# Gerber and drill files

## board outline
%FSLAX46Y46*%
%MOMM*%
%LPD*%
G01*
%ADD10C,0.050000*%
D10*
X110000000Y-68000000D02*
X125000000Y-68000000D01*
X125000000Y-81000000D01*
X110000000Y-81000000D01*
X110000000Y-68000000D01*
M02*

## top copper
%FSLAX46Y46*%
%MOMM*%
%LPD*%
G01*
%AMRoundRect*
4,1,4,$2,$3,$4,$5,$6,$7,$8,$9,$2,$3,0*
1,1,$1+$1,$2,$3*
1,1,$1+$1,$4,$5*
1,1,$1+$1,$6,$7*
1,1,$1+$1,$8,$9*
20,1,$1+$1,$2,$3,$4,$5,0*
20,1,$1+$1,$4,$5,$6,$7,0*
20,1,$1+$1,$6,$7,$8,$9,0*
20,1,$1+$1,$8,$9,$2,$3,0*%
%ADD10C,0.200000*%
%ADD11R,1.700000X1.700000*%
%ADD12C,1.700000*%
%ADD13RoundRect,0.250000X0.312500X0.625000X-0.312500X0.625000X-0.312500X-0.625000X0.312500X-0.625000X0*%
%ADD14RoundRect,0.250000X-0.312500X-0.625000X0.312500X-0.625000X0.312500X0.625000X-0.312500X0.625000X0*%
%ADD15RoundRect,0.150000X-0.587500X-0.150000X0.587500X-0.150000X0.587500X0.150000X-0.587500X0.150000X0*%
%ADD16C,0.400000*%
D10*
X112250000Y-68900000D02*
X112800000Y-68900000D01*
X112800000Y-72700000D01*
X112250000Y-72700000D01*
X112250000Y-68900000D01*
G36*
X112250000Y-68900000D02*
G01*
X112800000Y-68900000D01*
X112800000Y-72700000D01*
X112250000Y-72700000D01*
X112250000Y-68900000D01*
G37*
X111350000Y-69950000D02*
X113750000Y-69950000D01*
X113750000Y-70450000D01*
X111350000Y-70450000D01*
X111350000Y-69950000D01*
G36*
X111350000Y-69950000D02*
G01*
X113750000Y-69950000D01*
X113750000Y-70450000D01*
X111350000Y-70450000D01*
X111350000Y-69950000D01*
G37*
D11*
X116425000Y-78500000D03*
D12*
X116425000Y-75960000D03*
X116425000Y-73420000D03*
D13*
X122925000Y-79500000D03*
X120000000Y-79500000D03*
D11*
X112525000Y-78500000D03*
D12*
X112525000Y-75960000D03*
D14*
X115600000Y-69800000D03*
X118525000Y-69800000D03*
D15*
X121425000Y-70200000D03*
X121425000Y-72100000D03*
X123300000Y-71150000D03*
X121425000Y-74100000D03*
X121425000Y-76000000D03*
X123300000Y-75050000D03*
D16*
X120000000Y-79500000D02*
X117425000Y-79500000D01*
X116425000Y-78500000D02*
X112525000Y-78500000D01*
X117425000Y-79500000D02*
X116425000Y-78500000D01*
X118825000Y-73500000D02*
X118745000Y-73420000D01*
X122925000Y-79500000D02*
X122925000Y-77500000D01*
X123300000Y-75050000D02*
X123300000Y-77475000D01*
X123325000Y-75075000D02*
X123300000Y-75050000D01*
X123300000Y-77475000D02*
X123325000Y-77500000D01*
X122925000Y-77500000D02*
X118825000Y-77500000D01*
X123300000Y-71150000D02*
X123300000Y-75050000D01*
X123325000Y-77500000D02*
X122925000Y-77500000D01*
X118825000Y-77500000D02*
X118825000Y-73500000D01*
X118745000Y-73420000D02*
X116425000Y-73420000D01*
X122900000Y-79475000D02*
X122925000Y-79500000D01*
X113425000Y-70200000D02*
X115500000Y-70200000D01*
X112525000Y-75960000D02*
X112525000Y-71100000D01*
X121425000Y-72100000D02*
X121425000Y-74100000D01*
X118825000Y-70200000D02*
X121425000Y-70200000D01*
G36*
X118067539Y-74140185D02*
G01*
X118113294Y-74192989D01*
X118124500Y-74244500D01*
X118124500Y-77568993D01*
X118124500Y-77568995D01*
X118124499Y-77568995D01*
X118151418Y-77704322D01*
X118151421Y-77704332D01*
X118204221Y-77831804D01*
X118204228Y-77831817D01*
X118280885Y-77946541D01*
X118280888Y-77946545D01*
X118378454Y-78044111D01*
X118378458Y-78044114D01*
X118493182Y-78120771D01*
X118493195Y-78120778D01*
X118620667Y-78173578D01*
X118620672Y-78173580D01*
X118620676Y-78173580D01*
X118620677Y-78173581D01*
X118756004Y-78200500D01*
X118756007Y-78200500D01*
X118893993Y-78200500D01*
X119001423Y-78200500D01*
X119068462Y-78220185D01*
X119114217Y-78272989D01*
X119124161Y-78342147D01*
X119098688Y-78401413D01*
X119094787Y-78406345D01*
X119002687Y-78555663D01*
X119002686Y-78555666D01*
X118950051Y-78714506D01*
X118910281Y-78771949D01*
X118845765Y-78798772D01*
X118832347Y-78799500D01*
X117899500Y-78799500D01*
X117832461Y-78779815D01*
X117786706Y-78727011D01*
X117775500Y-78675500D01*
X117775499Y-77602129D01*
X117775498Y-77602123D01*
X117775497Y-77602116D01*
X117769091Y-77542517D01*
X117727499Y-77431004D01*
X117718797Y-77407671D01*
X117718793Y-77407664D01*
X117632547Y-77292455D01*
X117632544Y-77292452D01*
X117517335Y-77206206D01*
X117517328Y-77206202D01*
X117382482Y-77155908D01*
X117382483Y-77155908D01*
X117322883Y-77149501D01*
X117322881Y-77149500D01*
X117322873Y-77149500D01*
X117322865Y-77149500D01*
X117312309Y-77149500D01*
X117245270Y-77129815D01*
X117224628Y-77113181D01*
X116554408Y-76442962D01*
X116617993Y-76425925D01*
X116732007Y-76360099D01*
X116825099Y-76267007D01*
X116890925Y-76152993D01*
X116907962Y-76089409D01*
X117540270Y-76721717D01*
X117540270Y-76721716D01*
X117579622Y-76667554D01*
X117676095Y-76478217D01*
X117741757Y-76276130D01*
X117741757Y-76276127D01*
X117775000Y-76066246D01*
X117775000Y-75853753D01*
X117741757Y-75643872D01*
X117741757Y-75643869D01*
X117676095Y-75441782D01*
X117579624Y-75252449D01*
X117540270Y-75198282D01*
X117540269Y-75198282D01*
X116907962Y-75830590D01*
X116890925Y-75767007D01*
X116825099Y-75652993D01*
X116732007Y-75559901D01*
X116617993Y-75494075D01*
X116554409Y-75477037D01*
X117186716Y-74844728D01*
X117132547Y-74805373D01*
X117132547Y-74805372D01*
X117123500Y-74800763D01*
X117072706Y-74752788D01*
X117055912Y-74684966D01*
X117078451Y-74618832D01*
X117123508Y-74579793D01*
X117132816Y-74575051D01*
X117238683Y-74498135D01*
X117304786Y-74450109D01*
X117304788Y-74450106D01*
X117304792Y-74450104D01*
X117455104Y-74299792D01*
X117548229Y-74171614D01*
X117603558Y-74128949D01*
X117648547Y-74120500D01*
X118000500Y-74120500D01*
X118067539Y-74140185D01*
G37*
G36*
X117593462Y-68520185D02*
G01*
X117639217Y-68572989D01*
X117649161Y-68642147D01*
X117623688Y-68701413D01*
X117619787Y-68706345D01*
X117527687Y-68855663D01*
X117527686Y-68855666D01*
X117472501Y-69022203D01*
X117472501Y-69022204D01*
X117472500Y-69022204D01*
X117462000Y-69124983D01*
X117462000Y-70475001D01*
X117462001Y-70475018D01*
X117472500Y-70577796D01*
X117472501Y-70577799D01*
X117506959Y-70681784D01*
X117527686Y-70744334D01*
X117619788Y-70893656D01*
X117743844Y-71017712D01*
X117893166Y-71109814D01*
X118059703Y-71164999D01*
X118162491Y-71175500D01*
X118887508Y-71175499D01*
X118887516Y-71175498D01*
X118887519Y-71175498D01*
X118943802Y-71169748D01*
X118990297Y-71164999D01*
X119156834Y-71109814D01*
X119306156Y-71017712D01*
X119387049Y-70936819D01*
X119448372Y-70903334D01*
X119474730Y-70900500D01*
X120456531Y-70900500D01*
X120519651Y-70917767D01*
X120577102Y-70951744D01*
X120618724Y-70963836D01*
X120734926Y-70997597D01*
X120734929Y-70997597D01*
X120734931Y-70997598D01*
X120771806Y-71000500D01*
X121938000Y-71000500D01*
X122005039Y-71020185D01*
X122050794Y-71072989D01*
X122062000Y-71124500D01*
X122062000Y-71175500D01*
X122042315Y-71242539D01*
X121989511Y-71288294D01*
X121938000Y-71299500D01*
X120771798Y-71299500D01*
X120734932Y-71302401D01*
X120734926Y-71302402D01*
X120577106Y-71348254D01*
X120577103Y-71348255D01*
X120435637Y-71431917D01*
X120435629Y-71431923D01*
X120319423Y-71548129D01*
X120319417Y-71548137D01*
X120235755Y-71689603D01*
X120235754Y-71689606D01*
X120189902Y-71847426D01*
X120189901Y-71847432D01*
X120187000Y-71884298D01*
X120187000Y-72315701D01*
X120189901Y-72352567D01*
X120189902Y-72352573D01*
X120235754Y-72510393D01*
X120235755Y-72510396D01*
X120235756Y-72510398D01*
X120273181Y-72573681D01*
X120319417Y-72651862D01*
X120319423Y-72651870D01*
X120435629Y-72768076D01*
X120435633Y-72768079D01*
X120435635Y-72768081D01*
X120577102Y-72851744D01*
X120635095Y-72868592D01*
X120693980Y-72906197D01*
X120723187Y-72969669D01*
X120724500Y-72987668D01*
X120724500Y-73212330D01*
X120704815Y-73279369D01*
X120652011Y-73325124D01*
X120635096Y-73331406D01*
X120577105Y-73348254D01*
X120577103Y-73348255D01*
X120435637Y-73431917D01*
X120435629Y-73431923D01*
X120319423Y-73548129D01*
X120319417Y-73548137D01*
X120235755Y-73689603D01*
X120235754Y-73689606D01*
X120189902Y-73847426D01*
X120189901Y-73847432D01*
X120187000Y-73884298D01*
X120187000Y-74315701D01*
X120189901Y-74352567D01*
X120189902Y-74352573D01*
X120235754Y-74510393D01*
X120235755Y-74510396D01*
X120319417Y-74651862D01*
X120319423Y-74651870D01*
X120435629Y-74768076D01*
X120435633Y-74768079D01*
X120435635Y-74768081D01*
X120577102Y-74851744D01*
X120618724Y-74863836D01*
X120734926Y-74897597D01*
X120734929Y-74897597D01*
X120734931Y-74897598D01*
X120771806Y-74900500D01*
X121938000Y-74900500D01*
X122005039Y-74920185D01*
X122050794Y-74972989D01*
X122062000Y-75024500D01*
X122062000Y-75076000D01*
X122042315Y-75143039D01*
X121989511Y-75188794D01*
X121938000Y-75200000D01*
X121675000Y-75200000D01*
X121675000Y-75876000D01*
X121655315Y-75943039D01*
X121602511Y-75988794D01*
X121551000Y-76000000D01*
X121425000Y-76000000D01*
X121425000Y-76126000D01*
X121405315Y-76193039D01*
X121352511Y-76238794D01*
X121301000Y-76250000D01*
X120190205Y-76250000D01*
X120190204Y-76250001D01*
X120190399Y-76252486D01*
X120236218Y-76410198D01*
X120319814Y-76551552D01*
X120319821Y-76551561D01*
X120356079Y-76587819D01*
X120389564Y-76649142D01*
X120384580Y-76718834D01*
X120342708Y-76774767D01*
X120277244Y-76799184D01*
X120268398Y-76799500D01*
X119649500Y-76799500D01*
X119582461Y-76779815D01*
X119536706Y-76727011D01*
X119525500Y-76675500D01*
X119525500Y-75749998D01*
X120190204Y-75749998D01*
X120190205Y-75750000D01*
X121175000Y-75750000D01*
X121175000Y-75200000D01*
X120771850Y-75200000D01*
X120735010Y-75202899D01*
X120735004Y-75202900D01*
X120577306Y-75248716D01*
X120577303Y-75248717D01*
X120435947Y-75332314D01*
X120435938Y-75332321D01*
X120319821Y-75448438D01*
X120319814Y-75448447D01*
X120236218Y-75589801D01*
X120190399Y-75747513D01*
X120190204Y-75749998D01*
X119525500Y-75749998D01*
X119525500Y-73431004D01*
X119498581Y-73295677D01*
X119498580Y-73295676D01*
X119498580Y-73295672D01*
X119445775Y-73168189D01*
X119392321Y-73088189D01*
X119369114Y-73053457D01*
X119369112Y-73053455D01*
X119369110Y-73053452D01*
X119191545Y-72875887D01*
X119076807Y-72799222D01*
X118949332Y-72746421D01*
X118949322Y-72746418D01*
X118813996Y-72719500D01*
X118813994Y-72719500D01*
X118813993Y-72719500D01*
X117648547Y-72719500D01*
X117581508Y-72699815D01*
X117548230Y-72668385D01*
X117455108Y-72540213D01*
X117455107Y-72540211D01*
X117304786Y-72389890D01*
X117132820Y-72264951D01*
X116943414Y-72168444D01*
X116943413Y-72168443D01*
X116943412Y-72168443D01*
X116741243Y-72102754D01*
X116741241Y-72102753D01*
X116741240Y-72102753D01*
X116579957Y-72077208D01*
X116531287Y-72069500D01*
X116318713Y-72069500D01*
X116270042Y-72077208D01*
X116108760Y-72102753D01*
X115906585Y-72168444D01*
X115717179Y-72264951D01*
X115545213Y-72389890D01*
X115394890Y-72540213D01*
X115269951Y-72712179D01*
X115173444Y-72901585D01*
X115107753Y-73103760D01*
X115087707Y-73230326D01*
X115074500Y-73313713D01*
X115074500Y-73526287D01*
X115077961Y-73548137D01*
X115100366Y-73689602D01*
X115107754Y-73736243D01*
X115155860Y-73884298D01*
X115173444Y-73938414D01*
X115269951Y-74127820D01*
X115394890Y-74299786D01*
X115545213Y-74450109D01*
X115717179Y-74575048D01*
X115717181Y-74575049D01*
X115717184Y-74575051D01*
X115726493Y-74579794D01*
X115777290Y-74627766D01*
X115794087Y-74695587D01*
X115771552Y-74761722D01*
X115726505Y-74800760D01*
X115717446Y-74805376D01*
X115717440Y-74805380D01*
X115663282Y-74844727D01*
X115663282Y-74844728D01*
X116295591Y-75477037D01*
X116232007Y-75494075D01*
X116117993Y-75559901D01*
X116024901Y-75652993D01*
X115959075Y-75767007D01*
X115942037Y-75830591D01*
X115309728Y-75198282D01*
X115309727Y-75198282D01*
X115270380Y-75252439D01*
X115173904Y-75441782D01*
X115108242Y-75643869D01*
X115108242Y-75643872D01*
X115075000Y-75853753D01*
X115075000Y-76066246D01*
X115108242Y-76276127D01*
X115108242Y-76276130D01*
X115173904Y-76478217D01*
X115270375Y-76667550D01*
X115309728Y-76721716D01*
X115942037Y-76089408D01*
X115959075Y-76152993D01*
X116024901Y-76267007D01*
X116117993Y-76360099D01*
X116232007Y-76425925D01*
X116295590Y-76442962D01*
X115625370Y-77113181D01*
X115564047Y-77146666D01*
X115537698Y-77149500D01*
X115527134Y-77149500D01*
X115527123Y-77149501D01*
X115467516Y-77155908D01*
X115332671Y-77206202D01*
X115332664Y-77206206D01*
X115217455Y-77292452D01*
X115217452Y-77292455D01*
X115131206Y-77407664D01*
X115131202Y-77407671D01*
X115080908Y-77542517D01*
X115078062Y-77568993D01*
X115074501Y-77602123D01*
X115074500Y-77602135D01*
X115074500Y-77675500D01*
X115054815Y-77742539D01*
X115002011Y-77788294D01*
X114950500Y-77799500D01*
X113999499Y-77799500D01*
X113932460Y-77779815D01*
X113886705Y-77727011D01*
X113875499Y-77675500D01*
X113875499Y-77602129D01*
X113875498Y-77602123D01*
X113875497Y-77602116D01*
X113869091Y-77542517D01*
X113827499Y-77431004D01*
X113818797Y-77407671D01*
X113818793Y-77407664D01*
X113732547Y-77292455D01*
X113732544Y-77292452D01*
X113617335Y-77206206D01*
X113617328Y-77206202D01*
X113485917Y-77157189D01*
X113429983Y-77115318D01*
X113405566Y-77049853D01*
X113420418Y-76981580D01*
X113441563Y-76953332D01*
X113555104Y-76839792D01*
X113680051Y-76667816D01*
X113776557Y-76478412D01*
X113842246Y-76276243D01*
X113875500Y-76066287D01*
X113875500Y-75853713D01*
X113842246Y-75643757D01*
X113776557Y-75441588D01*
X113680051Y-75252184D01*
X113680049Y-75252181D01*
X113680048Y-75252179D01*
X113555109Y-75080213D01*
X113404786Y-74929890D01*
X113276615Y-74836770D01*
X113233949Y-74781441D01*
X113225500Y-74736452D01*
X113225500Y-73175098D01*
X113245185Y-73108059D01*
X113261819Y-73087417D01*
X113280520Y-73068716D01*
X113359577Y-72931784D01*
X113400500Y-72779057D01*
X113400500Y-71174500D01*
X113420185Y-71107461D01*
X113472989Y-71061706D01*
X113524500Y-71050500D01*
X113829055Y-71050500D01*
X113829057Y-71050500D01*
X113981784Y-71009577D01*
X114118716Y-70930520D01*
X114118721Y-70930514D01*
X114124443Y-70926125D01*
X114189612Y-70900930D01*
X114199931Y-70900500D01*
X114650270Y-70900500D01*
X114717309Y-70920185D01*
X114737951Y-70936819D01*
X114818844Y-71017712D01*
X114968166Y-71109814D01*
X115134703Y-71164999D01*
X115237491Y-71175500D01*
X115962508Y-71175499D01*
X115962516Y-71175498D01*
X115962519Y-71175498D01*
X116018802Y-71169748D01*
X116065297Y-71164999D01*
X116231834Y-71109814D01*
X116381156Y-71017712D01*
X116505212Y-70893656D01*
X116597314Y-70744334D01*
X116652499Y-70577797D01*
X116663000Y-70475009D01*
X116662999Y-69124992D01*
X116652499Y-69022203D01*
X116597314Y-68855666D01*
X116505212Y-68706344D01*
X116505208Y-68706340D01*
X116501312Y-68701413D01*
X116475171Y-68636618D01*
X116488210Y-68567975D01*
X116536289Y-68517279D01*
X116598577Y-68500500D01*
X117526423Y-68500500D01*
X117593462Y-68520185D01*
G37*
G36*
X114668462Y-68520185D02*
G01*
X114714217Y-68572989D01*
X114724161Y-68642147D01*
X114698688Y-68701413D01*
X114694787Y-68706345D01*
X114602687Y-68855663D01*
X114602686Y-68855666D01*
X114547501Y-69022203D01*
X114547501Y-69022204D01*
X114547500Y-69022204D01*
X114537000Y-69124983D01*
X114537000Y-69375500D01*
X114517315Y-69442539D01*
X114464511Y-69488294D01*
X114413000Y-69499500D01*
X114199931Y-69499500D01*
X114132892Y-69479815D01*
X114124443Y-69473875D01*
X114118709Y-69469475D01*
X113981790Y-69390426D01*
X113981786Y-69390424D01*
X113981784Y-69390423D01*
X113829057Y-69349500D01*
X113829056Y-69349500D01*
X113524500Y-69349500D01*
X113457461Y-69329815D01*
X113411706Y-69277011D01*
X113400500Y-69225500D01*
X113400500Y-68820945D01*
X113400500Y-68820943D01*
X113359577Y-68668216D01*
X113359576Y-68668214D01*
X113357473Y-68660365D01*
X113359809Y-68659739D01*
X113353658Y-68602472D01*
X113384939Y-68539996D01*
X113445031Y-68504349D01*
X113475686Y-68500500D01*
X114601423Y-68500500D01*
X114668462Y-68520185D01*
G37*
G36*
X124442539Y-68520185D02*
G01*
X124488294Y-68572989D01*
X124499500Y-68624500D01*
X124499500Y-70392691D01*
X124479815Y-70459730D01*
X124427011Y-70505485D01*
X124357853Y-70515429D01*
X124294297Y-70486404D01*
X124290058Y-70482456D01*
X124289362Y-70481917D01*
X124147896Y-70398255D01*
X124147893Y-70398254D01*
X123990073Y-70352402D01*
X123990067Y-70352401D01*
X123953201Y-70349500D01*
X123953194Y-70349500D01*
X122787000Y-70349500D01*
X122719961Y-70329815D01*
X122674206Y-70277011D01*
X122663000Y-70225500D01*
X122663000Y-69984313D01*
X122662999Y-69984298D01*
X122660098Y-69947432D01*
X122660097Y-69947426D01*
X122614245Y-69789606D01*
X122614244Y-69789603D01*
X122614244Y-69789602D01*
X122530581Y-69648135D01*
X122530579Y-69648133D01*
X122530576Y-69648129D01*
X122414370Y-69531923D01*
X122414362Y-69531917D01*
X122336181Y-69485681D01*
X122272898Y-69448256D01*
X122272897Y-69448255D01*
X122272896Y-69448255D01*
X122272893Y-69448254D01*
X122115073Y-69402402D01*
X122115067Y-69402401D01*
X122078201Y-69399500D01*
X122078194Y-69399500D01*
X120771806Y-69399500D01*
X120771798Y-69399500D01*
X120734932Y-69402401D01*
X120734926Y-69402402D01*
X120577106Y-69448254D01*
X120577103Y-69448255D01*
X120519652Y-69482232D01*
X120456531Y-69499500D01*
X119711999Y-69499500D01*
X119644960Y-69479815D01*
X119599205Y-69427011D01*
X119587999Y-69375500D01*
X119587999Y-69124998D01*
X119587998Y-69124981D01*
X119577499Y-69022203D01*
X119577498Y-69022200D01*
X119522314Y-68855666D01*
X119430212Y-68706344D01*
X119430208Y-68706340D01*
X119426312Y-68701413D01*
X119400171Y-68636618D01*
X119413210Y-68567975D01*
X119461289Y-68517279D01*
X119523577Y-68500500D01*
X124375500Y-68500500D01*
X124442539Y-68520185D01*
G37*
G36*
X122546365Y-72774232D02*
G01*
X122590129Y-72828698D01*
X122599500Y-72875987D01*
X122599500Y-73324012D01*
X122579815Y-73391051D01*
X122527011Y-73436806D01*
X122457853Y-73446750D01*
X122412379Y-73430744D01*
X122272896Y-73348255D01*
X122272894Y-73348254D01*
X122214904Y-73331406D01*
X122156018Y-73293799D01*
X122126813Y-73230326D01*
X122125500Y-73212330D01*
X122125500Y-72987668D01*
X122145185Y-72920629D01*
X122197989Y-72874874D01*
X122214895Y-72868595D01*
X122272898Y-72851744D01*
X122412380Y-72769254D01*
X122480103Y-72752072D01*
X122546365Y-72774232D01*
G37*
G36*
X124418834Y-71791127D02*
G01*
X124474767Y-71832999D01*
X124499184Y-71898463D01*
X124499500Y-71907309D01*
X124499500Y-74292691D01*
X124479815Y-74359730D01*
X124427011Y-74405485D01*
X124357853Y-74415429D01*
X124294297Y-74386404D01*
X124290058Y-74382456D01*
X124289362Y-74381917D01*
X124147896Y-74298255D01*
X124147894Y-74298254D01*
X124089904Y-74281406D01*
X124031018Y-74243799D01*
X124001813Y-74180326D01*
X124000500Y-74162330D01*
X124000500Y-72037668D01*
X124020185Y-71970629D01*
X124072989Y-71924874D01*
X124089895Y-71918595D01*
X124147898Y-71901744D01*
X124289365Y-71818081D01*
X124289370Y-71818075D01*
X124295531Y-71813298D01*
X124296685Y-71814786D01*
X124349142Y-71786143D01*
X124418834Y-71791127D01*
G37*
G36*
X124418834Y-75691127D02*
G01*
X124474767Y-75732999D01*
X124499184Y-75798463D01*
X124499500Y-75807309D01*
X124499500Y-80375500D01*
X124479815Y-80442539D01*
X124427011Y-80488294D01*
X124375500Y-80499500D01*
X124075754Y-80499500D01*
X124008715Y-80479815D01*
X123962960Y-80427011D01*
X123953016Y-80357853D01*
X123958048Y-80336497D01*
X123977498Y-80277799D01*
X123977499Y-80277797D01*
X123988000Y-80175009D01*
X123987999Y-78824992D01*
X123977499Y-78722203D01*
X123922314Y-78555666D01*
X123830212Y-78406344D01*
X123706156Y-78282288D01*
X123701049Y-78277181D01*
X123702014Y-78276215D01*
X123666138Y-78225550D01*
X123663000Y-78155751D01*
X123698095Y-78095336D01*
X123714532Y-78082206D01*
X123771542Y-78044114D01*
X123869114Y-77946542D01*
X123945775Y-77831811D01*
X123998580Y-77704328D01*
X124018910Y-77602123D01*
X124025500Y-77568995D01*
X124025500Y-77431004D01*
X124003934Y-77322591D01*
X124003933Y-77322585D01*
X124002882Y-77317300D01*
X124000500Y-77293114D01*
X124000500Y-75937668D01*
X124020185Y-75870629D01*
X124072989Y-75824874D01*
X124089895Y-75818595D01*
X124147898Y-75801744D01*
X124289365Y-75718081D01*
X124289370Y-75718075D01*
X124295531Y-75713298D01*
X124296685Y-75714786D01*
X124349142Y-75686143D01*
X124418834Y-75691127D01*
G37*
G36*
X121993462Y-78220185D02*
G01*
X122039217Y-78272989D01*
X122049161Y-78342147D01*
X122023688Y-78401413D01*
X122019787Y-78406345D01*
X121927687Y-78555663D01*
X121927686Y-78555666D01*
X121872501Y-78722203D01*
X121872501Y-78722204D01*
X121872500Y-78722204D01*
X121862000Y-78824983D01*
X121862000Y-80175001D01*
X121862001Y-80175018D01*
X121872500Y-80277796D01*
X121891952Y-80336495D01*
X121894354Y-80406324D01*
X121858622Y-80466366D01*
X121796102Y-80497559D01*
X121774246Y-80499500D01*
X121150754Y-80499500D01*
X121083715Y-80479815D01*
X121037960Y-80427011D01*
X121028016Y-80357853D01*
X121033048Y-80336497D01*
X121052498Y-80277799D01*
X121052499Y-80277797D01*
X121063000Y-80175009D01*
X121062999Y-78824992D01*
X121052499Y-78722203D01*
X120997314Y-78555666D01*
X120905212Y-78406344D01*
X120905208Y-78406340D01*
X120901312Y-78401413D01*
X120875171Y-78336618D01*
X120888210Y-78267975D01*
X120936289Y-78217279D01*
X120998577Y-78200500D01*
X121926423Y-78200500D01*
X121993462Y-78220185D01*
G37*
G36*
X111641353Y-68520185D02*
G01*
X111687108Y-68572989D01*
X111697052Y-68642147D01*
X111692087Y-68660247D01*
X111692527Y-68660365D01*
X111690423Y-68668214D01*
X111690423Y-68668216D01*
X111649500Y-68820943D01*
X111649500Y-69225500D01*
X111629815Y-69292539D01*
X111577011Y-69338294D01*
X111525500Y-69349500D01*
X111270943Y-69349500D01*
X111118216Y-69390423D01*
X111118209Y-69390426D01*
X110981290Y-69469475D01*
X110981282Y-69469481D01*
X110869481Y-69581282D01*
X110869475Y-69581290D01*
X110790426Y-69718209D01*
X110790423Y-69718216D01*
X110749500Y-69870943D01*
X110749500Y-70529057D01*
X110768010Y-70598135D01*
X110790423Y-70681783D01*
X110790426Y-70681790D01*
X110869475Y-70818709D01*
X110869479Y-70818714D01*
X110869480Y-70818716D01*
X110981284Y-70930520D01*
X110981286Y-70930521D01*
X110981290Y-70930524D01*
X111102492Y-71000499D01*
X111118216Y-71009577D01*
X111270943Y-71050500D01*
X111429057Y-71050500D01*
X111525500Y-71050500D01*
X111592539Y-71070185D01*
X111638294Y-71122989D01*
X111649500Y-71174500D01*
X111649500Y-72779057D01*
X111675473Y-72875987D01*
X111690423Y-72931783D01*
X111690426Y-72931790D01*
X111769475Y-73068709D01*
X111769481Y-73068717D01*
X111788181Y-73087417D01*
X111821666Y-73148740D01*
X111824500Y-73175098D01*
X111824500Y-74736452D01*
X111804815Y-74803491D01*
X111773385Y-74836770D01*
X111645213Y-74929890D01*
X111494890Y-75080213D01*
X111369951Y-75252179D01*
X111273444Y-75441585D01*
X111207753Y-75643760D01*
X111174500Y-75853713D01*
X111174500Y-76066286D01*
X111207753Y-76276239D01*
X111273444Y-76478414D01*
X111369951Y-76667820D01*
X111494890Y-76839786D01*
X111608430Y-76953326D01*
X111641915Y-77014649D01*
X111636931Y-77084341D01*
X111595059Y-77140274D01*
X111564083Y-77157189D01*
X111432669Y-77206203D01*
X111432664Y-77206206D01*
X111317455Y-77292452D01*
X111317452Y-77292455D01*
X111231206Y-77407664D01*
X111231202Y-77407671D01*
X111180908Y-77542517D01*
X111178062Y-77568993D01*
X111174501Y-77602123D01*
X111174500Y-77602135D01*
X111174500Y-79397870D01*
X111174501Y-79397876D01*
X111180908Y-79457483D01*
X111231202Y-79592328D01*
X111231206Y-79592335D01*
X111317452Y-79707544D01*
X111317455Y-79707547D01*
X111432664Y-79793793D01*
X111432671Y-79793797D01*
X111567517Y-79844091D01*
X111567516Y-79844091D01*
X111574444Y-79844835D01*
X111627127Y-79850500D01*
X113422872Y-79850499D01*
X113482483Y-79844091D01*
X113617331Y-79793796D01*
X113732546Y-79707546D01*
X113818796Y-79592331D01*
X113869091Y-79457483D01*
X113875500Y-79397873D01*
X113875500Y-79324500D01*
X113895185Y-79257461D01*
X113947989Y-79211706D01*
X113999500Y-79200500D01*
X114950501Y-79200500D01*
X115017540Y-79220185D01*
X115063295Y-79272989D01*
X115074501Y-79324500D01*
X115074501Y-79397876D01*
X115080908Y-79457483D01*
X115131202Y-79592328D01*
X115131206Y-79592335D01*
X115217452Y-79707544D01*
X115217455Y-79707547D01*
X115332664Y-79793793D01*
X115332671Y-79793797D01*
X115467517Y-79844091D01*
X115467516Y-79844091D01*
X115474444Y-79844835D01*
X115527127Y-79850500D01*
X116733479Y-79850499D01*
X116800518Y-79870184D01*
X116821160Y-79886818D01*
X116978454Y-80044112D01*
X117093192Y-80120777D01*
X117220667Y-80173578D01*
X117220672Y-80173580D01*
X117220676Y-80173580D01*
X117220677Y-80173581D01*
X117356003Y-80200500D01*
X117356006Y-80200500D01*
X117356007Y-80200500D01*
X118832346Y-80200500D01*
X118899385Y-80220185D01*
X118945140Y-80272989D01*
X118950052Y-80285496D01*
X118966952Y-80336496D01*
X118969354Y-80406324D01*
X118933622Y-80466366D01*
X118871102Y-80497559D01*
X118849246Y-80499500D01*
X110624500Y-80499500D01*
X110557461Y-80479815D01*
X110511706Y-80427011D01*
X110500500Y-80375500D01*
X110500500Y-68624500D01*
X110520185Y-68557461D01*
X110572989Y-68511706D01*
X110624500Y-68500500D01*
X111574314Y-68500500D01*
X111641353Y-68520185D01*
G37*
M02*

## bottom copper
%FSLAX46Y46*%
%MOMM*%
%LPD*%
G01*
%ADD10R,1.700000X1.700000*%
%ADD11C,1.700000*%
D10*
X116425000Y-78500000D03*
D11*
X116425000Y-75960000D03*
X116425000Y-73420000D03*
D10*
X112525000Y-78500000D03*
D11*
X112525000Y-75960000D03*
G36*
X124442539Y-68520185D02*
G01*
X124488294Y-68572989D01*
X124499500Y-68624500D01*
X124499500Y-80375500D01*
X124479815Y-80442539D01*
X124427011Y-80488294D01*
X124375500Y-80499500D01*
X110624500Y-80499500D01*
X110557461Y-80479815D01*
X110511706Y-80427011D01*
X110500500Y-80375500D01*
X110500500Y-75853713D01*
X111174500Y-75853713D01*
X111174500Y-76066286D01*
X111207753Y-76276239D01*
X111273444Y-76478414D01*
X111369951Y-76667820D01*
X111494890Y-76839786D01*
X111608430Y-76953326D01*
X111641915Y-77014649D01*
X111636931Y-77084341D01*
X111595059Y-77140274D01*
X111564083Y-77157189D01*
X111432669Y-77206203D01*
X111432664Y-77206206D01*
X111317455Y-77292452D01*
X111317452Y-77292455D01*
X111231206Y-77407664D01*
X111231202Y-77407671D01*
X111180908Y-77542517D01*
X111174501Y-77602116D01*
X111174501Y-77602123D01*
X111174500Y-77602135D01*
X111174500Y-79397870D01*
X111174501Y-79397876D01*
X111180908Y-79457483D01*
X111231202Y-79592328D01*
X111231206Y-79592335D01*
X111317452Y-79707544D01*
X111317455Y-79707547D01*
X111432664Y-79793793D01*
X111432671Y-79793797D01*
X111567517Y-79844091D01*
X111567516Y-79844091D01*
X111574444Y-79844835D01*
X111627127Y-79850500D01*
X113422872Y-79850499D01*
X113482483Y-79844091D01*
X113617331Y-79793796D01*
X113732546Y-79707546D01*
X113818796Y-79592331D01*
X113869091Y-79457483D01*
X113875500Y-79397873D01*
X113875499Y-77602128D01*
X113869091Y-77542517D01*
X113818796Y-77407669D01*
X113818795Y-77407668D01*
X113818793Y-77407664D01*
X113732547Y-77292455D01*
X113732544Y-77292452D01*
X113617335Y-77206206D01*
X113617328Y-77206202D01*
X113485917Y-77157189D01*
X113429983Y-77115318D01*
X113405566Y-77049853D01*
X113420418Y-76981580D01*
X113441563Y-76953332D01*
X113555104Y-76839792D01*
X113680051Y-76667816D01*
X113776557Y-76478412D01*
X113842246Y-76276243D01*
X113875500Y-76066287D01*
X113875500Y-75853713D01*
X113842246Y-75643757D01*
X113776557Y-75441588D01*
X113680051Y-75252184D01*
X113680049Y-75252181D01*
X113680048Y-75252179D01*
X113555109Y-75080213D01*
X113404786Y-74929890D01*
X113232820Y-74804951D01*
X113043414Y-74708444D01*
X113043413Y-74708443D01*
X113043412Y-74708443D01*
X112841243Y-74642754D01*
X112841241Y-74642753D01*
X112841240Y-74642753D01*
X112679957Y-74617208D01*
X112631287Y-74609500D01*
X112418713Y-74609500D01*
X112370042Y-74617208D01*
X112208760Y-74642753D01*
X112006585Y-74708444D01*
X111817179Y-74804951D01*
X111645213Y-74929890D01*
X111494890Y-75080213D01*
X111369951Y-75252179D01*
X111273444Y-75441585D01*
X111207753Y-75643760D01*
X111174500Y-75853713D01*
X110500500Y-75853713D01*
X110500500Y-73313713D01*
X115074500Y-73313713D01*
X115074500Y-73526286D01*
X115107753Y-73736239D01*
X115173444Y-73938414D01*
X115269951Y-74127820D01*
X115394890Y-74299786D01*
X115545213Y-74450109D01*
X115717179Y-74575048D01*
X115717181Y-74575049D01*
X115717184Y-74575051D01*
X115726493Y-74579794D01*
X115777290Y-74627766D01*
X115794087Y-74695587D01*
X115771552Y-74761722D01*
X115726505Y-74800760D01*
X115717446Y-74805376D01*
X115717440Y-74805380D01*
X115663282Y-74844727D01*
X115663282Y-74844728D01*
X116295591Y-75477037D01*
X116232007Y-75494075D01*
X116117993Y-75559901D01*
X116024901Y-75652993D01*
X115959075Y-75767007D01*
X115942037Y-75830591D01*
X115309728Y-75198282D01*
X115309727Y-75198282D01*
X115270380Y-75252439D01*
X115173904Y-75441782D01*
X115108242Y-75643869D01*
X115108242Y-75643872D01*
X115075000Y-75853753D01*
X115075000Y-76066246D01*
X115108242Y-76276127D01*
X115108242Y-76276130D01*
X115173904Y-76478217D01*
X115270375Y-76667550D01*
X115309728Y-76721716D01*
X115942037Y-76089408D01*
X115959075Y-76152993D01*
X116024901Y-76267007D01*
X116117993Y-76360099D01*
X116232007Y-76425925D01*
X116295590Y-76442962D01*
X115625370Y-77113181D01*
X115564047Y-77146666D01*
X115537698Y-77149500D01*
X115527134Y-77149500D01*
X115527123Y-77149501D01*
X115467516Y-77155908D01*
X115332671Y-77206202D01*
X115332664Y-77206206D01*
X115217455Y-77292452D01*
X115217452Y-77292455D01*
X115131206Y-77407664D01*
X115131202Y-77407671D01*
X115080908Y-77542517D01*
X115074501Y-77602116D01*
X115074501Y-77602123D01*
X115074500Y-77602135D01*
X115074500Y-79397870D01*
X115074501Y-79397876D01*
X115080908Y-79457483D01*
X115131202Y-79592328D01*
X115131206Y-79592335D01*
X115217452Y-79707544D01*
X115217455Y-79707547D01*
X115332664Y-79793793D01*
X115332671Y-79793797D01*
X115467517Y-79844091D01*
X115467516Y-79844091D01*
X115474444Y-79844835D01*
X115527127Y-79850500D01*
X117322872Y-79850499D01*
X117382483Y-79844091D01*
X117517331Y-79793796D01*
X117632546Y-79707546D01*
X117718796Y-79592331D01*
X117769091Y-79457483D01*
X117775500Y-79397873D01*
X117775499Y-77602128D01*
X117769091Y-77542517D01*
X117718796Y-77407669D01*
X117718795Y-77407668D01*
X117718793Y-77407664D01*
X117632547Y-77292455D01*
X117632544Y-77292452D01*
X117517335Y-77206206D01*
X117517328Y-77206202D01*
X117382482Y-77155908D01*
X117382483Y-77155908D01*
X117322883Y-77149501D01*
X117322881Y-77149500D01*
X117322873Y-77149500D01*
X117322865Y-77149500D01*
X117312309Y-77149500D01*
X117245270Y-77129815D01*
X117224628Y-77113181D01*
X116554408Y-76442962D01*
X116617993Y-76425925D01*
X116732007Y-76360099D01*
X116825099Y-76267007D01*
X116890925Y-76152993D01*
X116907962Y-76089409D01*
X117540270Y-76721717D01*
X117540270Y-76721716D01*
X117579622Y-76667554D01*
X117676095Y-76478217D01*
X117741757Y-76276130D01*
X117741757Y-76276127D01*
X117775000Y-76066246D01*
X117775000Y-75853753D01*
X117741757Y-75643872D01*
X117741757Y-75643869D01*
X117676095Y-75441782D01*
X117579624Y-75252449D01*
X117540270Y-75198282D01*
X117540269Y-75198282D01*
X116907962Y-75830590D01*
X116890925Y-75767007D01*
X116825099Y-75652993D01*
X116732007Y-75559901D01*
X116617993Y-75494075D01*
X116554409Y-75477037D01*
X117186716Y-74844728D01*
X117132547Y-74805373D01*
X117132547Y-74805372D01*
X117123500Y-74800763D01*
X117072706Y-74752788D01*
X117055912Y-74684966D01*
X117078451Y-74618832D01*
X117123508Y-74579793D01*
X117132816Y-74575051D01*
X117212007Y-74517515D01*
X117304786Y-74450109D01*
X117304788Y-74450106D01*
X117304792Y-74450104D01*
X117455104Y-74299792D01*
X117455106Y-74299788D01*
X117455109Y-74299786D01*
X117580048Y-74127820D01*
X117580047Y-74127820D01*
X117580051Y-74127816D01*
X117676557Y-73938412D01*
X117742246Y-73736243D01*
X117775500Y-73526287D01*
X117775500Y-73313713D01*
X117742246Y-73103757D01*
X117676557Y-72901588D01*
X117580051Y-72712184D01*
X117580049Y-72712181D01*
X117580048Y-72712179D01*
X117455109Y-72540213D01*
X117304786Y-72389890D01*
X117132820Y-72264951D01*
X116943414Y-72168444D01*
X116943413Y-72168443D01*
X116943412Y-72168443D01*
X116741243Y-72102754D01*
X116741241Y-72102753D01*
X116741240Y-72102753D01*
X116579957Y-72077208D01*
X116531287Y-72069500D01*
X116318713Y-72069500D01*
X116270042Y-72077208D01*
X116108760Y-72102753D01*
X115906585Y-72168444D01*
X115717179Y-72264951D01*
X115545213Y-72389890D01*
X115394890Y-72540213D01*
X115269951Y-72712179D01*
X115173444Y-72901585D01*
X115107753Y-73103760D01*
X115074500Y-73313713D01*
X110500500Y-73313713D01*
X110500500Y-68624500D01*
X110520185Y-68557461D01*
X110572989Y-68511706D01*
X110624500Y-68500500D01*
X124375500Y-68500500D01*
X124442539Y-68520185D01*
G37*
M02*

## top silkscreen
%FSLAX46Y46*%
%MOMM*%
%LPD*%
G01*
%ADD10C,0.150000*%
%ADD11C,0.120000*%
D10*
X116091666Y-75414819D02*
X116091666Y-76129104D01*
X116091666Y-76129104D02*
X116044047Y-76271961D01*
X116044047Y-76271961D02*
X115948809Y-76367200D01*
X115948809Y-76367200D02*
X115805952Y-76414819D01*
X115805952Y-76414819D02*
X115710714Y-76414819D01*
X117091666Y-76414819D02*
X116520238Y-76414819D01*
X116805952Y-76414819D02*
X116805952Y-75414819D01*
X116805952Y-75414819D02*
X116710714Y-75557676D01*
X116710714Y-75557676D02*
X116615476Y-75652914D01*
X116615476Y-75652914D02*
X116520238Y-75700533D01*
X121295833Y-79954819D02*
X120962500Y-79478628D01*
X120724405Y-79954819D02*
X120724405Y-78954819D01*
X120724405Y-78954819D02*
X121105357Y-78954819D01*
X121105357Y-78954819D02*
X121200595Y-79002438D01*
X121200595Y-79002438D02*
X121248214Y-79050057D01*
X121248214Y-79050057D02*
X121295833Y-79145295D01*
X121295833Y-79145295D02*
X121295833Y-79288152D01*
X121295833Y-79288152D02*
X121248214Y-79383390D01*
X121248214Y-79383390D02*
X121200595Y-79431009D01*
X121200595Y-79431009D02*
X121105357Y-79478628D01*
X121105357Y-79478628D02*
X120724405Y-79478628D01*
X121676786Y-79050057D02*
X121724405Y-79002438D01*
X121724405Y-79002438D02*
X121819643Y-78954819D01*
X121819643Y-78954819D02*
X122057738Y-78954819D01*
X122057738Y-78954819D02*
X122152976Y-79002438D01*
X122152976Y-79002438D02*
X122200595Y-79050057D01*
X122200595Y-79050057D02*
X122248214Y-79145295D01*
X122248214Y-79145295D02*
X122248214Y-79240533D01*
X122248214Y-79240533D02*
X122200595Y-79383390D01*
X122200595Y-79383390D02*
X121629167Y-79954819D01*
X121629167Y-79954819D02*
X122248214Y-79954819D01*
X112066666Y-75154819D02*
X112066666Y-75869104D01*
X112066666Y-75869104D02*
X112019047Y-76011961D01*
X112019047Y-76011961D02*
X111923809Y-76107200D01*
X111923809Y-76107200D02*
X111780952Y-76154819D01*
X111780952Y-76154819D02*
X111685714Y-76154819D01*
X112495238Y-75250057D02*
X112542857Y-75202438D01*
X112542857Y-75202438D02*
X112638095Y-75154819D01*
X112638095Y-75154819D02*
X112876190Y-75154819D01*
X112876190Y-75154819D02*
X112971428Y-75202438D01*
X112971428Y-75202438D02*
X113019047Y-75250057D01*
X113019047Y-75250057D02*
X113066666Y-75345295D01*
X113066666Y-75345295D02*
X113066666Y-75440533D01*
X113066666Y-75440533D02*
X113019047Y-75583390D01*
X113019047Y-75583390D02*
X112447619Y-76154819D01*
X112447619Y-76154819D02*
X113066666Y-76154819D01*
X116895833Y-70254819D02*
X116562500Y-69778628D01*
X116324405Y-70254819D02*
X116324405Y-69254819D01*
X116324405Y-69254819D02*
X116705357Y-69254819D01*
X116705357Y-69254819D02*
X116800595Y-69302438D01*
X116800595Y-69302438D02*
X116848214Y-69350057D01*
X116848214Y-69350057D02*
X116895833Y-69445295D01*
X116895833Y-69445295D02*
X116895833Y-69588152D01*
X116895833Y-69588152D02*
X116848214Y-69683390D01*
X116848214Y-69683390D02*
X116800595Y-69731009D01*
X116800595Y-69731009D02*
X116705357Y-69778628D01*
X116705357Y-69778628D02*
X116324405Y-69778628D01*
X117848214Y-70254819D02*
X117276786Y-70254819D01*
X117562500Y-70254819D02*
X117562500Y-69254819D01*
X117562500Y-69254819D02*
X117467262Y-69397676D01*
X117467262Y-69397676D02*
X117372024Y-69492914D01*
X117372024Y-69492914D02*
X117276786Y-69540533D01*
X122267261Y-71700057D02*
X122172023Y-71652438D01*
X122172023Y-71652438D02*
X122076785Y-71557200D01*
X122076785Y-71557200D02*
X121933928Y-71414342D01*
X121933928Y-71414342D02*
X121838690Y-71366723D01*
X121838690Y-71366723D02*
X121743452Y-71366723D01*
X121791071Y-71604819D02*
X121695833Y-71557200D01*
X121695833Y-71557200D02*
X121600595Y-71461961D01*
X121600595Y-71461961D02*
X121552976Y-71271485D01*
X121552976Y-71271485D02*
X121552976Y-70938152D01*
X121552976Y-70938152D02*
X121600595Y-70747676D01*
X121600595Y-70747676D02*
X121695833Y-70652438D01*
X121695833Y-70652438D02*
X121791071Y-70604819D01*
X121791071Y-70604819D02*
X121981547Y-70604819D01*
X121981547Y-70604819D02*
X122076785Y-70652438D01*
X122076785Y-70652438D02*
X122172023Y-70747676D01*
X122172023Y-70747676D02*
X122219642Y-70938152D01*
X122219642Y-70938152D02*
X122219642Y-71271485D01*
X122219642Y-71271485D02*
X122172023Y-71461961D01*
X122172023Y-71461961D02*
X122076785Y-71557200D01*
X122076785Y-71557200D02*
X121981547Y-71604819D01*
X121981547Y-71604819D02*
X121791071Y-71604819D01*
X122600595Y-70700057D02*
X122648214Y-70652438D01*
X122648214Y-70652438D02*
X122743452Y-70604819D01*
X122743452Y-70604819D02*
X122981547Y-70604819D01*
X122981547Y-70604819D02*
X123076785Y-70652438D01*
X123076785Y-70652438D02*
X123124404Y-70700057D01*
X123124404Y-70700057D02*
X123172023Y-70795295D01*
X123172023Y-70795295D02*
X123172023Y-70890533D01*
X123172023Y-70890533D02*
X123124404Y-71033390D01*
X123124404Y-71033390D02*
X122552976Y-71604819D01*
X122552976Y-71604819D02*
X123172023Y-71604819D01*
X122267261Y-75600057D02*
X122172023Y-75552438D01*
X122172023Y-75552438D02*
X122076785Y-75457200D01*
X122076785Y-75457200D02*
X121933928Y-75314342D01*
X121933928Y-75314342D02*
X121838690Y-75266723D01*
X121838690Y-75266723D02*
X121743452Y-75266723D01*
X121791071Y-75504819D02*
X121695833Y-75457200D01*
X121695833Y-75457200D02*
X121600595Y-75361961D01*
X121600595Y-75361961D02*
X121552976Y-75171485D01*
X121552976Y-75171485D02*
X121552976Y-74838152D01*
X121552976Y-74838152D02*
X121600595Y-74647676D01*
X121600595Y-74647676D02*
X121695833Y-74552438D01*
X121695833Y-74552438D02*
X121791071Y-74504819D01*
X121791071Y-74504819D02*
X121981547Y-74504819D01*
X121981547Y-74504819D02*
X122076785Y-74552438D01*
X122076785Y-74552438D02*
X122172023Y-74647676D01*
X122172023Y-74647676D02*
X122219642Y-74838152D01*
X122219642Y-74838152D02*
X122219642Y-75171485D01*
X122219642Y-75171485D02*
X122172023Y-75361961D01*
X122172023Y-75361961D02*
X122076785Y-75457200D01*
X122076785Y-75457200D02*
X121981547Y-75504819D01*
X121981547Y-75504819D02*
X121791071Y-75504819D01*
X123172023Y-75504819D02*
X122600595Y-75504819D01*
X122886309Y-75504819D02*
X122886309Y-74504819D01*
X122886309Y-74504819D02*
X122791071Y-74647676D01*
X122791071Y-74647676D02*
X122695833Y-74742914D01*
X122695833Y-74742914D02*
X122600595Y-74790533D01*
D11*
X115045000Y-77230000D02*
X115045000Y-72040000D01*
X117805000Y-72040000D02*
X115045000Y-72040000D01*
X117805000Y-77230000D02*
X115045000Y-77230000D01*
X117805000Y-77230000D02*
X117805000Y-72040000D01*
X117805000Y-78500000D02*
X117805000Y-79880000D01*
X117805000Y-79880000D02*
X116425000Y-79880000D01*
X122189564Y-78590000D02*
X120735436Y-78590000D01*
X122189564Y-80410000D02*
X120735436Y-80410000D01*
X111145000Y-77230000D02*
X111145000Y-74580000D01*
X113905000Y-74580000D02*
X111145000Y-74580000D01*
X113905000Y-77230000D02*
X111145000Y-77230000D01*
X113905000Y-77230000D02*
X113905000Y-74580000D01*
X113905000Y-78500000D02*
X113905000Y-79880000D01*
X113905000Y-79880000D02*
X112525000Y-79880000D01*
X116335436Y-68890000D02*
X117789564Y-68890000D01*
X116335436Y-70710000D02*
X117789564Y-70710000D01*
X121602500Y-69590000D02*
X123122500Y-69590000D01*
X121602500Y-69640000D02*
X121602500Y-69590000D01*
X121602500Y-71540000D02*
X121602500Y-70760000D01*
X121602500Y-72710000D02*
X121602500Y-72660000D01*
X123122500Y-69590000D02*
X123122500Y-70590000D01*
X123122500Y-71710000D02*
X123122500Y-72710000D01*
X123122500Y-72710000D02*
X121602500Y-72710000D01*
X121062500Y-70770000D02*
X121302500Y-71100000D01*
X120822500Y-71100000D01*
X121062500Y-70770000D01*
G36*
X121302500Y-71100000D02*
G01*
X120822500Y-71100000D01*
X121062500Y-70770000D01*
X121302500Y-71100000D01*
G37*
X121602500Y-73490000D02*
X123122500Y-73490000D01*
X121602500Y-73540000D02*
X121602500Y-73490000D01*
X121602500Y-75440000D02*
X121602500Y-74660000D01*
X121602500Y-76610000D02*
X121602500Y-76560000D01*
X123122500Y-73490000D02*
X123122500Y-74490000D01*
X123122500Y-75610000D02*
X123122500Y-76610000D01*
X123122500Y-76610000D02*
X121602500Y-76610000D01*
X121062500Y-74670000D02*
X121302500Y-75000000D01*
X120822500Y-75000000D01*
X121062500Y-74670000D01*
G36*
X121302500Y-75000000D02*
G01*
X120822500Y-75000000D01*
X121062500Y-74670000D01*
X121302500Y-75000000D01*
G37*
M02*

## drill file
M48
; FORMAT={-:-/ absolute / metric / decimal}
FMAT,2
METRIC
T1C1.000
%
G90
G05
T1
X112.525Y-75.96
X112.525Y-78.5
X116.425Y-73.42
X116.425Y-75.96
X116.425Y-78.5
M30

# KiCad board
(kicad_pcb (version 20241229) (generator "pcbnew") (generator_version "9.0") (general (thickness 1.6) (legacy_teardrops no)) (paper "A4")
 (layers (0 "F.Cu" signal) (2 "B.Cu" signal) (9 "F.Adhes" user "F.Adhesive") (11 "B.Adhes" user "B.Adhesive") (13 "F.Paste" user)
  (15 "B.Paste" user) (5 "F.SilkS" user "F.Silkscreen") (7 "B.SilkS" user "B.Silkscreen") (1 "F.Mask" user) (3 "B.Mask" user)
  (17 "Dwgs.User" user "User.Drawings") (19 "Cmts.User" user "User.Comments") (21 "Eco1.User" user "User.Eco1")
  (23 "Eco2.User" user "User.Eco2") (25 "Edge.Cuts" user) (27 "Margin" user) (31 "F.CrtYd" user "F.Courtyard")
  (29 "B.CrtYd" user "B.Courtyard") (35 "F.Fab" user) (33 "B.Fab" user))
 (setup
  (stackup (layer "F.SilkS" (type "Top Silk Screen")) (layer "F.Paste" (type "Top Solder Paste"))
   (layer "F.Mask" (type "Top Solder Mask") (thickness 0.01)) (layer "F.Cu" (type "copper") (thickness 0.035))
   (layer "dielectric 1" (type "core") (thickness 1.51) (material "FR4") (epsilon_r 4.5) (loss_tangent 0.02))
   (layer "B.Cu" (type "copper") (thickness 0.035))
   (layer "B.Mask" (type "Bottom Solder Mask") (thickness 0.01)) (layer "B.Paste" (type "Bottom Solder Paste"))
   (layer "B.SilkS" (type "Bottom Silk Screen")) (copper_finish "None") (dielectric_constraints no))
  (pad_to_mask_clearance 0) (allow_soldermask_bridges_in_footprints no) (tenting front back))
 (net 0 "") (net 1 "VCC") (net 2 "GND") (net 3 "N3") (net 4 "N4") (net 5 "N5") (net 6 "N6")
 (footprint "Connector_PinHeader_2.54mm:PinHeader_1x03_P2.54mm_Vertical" (layer "F.Cu") (at 116.425 78.5 180)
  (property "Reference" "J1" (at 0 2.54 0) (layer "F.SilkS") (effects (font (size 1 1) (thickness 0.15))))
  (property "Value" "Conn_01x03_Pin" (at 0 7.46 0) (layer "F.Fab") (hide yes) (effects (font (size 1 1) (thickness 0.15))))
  (fp_line (start 1.38 1.27) (end 1.38 6.46) (stroke (width 0.12) (type solid)) (layer "F.SilkS"))
  (fp_line (start -1.38 6.46) (end 1.38 6.46) (stroke (width 0.12) (type solid)) (layer "F.SilkS"))
  (fp_line (start -1.38 1.27) (end 1.38 1.27) (stroke (width 0.12) (type solid)) (layer "F.SilkS"))
  (fp_line (start -1.38 1.27) (end -1.38 6.46) (stroke (width 0.12) (type solid)) (layer "F.SilkS"))
  (fp_line (start -1.38 0) (end -1.38 -1.38) (stroke (width 0.12) (type solid)) (layer "F.SilkS"))
  (fp_line (start -1.38 -1.38) (end 0 -1.38) (stroke (width 0.12) (type solid)) (layer "F.SilkS"))
  (pad "1" thru_hole rect (at 0 0 180) (size 1.7 1.7) (drill 1) (layers "*.Cu" "*.Mask") (remove_unused_layers no) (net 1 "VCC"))
  (pad "2" thru_hole circle (at 0 2.54 180) (size 1.7 1.7) (drill 1) (layers "*.Cu" "*.Mask") (remove_unused_layers no) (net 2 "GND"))
  (pad "3" thru_hole circle (at 0 5.08 180) (size 1.7 1.7) (drill 1) (layers "*.Cu" "*.Mask") (remove_unused_layers no) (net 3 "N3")))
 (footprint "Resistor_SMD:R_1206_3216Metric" (layer "F.Cu") (at 121.4625 79.5 180)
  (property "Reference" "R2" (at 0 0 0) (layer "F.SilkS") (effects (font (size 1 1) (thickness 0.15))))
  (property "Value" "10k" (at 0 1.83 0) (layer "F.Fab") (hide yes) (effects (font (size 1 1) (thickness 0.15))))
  (fp_line (start -0.727064 0.91) (end 0.727064 0.91) (stroke (width 0.12) (type solid)) (layer "F.SilkS"))
  (fp_line (start -0.727064 -0.91) (end 0.727064 -0.91) (stroke (width 0.12) (type solid)) (layer "F.SilkS"))
  (pad "1" smd roundrect (at -1.4625 0 180) (size 1.125 1.75) (layers "F.Cu" "F.Mask" "F.Paste") (roundrect_rratio 0.222222) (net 3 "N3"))
  (pad "2" smd roundrect (at 1.4625 0 180) (size 1.125 1.75) (layers "F.Cu" "F.Mask" "F.Paste") (roundrect_rratio 0.222222) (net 1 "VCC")))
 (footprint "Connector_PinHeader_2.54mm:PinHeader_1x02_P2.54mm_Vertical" (layer "F.Cu") (at 112.525 78.5 180)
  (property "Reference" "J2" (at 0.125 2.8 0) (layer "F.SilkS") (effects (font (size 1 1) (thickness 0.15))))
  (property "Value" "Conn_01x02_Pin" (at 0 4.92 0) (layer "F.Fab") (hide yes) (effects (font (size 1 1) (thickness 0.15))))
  (fp_line (start 1.38 1.27) (end 1.38 3.92) (stroke (width 0.12) (type solid)) (layer "F.SilkS"))
  (fp_line (start -1.38 3.92) (end 1.38 3.92) (stroke (width 0.12) (type solid)) (layer "F.SilkS"))
  (fp_line (start -1.38 1.27) (end 1.38 1.27) (stroke (width 0.12) (type solid)) (layer "F.SilkS"))
  (fp_line (start -1.38 1.27) (end -1.38 3.92) (stroke (width 0.12) (type solid)) (layer "F.SilkS"))
  (fp_line (start -1.38 0) (end -1.38 -1.38) (stroke (width 0.12) (type solid)) (layer "F.SilkS"))
  (fp_line (start -1.38 -1.38) (end 0 -1.38) (stroke (width 0.12) (type solid)) (layer "F.SilkS"))
  (pad "1" thru_hole rect (at 0 0 180) (size 1.7 1.7) (drill 1) (layers "*.Cu" "*.Mask") (remove_unused_layers no) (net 1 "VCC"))
  (pad "2" thru_hole circle (at 0 2.54 180) (size 1.7 1.7) (drill 1) (layers "*.Cu" "*.Mask") (remove_unused_layers no) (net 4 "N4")))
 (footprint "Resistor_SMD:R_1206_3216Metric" (layer "F.Cu") (at 117.0625 69.8)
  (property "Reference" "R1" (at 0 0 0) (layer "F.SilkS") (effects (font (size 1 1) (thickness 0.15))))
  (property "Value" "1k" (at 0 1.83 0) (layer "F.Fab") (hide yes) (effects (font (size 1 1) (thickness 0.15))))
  (fp_line (start -0.727064 -0.91) (end 0.727064 -0.91) (stroke (width 0.12) (type solid)) (layer "F.SilkS"))
  (fp_line (start -0.727064 0.91) (end 0.727064 0.91) (stroke (width 0.12) (type solid)) (layer "F.SilkS"))
  (pad "1" smd roundrect (at -1.4625 0) (size 1.125 1.75) (layers "F.Cu" "F.Mask" "F.Paste") (roundrect_rratio 0.222222) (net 4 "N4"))
  (pad "2" smd roundrect (at 1.4625 0) (size 1.125 1.75) (layers "F.Cu" "F.Mask" "F.Paste") (roundrect_rratio 0.222222) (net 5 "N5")))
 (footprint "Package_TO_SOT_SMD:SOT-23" (layer "F.Cu") (at 122.3625 71.15)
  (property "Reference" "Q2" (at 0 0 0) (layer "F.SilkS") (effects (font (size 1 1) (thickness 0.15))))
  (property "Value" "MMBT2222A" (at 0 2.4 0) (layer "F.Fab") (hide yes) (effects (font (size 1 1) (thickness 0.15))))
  (fp_line (start -0.76 -1.56) (end 0.76 -1.56) (stroke (width 0.12) (type solid)) (layer "F.SilkS"))
  (fp_line (start -0.76 -1.51) (end -0.76 -1.56) (stroke (width 0.12) (type solid)) (layer "F.SilkS"))
  (fp_line (start -0.76 0.39) (end -0.76 -0.39) (stroke (width 0.12) (type solid)) (layer "F.SilkS"))
  (fp_line (start -0.76 1.56) (end -0.76 1.51) (stroke (width 0.12) (type solid)) (layer "F.SilkS"))
  (fp_line (start 0.76 -1.56) (end 0.76 -0.56) (stroke (width 0.12) (type solid)) (layer "F.SilkS"))
  (fp_line (start 0.76 0.56) (end 0.76 1.56) (stroke (width 0.12) (type solid)) (layer "F.SilkS"))
  (fp_line (start 0.76 1.56) (end -0.76 1.56) (stroke (width 0.12) (type solid)) (layer "F.SilkS"))
  (fp_poly (pts (xy -1.3 -0.38) (xy -1.06 -0.05) (xy -1.54 -0.05)) (stroke (width 0.12) (type solid)) (fill yes) (layer "F.SilkS"))
  (pad "1" smd roundrect (at -0.9375 -0.95) (size 1.475 0.6) (layers "F.Cu" "F.Mask" "F.Paste") (roundrect_rratio 0.25) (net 5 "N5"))
  (pad "2" smd roundrect (at -0.9375 0.95) (size 1.475 0.6) (layers "F.Cu" "F.Mask" "F.Paste") (roundrect_rratio 0.25) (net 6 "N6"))
  (pad "3" smd roundrect (at 0.9375 0) (size 1.475 0.6) (layers "F.Cu" "F.Mask" "F.Paste") (roundrect_rratio 0.25) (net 3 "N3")))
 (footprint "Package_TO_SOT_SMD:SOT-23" (layer "F.Cu") (at 122.3625 75.05)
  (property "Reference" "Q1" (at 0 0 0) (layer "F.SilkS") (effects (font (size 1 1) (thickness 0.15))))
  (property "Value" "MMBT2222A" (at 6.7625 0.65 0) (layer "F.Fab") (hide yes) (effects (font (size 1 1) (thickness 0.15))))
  (fp_line (start -0.76 -1.56) (end 0.76 -1.56) (stroke (width 0.12) (type solid)) (layer "F.SilkS"))
  (fp_line (start -0.76 -1.51) (end -0.76 -1.56) (stroke (width 0.12) (type solid)) (layer "F.SilkS"))
  (fp_line (start -0.76 0.39) (end -0.76 -0.39) (stroke (width 0.12) (type solid)) (layer "F.SilkS"))
  (fp_line (start -0.76 1.56) (end -0.76 1.51) (stroke (width 0.12) (type solid)) (layer "F.SilkS"))
  (fp_line (start 0.76 -1.56) (end 0.76 -0.56) (stroke (width 0.12) (type solid)) (layer "F.SilkS"))
  (fp_line (start 0.76 0.56) (end 0.76 1.56) (stroke (width 0.12) (type solid)) (layer "F.SilkS"))
  (fp_line (start 0.76 1.56) (end -0.76 1.56) (stroke (width 0.12) (type solid)) (layer "F.SilkS"))
  (fp_poly (pts (xy -1.3 -0.38) (xy -1.06 -0.05) (xy -1.54 -0.05)) (stroke (width 0.12) (type solid)) (fill yes) (layer "F.SilkS"))
  (pad "1" smd roundrect (at -0.9375 -0.95) (size 1.475 0.6) (layers "F.Cu" "F.Mask" "F.Paste") (roundrect_rratio 0.25) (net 6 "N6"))
  (pad "2" smd roundrect (at -0.9375 0.95) (size 1.475 0.6) (layers "F.Cu" "F.Mask" "F.Paste") (roundrect_rratio 0.25) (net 2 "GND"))
  (pad "3" smd roundrect (at 0.9375 0) (size 1.475 0.6) (layers "F.Cu" "F.Mask" "F.Paste") (roundrect_rratio 0.25) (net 3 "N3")))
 (gr_rect (start 112.25 68.9) (end 112.8 72.7) (stroke (width 0.2) (type solid)) (fill yes) (layer "F.Cu") (net 4))
 (gr_rect (start 111.35 69.95) (end 113.75 70.45) (stroke (width 0.2) (type solid)) (fill yes) (layer "F.Cu") (net 4))
 (gr_rect (start 110 68) (end 125 81) (stroke (width 0.05) (type default)) (fill no) (layer "Edge.Cuts"))
 (segment (start 120 79.5) (end 117.425 79.5) (width 0.4) (layer "F.Cu") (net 1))
 (segment (start 116.425 78.5) (end 112.525 78.5) (width 0.4) (layer "F.Cu") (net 1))
 (segment (start 117.425 79.5) (end 116.425 78.5) (width 0.4) (layer "F.Cu") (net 1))
 (segment (start 118.825 73.5) (end 118.745 73.42) (width 0.4) (layer "F.Cu") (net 3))
 (segment (start 122.925 79.5) (end 122.925 77.5) (width 0.4) (layer "F.Cu") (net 3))
 (segment (start 123.3 75.05) (end 123.3 77.475) (width 0.4) (layer "F.Cu") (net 3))
 (segment (start 123.325 75.075) (end 123.3 75.05) (width 0.4) (layer "F.Cu") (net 3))
 (segment (start 123.3 77.475) (end 123.325 77.5) (width 0.4) (layer "F.Cu") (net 3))
 (segment (start 122.925 77.5) (end 118.825 77.5) (width 0.4) (layer "F.Cu") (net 3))
 (segment (start 123.3 71.15) (end 123.3 75.05) (width 0.4) (layer "F.Cu") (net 3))
 (segment (start 123.325 77.5) (end 122.925 77.5) (width 0.4) (layer "F.Cu") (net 3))
 (segment (start 118.825 77.5) (end 118.825 73.5) (width 0.4) (layer "F.Cu") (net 3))
 (segment (start 118.745 73.42) (end 116.425 73.42) (width 0.4) (layer "F.Cu") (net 3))
 (segment (start 122.9 79.475) (end 122.925 79.5) (width 0.4) (layer "F.Cu") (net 3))
 (segment (start 113.425 70.2) (end 115.5 70.2) (width 0.4) (layer "F.Cu") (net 4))
 (segment (start 112.525 75.96) (end 112.525 71.1) (width 0.4) (layer "F.Cu") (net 4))
 (segment (start 121.425 72.1) (end 121.425 74.1) (width 0.4) (layer "F.Cu") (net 6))
 (segment (start 118.825 70.2) (end 121.425 70.2) (width 0.4) (layer "F.Cu") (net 5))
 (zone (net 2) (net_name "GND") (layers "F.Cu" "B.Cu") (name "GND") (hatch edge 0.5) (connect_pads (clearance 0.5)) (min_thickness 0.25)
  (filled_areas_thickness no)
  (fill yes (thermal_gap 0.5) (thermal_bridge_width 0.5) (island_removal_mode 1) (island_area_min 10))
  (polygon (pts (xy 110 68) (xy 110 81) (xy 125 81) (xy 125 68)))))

